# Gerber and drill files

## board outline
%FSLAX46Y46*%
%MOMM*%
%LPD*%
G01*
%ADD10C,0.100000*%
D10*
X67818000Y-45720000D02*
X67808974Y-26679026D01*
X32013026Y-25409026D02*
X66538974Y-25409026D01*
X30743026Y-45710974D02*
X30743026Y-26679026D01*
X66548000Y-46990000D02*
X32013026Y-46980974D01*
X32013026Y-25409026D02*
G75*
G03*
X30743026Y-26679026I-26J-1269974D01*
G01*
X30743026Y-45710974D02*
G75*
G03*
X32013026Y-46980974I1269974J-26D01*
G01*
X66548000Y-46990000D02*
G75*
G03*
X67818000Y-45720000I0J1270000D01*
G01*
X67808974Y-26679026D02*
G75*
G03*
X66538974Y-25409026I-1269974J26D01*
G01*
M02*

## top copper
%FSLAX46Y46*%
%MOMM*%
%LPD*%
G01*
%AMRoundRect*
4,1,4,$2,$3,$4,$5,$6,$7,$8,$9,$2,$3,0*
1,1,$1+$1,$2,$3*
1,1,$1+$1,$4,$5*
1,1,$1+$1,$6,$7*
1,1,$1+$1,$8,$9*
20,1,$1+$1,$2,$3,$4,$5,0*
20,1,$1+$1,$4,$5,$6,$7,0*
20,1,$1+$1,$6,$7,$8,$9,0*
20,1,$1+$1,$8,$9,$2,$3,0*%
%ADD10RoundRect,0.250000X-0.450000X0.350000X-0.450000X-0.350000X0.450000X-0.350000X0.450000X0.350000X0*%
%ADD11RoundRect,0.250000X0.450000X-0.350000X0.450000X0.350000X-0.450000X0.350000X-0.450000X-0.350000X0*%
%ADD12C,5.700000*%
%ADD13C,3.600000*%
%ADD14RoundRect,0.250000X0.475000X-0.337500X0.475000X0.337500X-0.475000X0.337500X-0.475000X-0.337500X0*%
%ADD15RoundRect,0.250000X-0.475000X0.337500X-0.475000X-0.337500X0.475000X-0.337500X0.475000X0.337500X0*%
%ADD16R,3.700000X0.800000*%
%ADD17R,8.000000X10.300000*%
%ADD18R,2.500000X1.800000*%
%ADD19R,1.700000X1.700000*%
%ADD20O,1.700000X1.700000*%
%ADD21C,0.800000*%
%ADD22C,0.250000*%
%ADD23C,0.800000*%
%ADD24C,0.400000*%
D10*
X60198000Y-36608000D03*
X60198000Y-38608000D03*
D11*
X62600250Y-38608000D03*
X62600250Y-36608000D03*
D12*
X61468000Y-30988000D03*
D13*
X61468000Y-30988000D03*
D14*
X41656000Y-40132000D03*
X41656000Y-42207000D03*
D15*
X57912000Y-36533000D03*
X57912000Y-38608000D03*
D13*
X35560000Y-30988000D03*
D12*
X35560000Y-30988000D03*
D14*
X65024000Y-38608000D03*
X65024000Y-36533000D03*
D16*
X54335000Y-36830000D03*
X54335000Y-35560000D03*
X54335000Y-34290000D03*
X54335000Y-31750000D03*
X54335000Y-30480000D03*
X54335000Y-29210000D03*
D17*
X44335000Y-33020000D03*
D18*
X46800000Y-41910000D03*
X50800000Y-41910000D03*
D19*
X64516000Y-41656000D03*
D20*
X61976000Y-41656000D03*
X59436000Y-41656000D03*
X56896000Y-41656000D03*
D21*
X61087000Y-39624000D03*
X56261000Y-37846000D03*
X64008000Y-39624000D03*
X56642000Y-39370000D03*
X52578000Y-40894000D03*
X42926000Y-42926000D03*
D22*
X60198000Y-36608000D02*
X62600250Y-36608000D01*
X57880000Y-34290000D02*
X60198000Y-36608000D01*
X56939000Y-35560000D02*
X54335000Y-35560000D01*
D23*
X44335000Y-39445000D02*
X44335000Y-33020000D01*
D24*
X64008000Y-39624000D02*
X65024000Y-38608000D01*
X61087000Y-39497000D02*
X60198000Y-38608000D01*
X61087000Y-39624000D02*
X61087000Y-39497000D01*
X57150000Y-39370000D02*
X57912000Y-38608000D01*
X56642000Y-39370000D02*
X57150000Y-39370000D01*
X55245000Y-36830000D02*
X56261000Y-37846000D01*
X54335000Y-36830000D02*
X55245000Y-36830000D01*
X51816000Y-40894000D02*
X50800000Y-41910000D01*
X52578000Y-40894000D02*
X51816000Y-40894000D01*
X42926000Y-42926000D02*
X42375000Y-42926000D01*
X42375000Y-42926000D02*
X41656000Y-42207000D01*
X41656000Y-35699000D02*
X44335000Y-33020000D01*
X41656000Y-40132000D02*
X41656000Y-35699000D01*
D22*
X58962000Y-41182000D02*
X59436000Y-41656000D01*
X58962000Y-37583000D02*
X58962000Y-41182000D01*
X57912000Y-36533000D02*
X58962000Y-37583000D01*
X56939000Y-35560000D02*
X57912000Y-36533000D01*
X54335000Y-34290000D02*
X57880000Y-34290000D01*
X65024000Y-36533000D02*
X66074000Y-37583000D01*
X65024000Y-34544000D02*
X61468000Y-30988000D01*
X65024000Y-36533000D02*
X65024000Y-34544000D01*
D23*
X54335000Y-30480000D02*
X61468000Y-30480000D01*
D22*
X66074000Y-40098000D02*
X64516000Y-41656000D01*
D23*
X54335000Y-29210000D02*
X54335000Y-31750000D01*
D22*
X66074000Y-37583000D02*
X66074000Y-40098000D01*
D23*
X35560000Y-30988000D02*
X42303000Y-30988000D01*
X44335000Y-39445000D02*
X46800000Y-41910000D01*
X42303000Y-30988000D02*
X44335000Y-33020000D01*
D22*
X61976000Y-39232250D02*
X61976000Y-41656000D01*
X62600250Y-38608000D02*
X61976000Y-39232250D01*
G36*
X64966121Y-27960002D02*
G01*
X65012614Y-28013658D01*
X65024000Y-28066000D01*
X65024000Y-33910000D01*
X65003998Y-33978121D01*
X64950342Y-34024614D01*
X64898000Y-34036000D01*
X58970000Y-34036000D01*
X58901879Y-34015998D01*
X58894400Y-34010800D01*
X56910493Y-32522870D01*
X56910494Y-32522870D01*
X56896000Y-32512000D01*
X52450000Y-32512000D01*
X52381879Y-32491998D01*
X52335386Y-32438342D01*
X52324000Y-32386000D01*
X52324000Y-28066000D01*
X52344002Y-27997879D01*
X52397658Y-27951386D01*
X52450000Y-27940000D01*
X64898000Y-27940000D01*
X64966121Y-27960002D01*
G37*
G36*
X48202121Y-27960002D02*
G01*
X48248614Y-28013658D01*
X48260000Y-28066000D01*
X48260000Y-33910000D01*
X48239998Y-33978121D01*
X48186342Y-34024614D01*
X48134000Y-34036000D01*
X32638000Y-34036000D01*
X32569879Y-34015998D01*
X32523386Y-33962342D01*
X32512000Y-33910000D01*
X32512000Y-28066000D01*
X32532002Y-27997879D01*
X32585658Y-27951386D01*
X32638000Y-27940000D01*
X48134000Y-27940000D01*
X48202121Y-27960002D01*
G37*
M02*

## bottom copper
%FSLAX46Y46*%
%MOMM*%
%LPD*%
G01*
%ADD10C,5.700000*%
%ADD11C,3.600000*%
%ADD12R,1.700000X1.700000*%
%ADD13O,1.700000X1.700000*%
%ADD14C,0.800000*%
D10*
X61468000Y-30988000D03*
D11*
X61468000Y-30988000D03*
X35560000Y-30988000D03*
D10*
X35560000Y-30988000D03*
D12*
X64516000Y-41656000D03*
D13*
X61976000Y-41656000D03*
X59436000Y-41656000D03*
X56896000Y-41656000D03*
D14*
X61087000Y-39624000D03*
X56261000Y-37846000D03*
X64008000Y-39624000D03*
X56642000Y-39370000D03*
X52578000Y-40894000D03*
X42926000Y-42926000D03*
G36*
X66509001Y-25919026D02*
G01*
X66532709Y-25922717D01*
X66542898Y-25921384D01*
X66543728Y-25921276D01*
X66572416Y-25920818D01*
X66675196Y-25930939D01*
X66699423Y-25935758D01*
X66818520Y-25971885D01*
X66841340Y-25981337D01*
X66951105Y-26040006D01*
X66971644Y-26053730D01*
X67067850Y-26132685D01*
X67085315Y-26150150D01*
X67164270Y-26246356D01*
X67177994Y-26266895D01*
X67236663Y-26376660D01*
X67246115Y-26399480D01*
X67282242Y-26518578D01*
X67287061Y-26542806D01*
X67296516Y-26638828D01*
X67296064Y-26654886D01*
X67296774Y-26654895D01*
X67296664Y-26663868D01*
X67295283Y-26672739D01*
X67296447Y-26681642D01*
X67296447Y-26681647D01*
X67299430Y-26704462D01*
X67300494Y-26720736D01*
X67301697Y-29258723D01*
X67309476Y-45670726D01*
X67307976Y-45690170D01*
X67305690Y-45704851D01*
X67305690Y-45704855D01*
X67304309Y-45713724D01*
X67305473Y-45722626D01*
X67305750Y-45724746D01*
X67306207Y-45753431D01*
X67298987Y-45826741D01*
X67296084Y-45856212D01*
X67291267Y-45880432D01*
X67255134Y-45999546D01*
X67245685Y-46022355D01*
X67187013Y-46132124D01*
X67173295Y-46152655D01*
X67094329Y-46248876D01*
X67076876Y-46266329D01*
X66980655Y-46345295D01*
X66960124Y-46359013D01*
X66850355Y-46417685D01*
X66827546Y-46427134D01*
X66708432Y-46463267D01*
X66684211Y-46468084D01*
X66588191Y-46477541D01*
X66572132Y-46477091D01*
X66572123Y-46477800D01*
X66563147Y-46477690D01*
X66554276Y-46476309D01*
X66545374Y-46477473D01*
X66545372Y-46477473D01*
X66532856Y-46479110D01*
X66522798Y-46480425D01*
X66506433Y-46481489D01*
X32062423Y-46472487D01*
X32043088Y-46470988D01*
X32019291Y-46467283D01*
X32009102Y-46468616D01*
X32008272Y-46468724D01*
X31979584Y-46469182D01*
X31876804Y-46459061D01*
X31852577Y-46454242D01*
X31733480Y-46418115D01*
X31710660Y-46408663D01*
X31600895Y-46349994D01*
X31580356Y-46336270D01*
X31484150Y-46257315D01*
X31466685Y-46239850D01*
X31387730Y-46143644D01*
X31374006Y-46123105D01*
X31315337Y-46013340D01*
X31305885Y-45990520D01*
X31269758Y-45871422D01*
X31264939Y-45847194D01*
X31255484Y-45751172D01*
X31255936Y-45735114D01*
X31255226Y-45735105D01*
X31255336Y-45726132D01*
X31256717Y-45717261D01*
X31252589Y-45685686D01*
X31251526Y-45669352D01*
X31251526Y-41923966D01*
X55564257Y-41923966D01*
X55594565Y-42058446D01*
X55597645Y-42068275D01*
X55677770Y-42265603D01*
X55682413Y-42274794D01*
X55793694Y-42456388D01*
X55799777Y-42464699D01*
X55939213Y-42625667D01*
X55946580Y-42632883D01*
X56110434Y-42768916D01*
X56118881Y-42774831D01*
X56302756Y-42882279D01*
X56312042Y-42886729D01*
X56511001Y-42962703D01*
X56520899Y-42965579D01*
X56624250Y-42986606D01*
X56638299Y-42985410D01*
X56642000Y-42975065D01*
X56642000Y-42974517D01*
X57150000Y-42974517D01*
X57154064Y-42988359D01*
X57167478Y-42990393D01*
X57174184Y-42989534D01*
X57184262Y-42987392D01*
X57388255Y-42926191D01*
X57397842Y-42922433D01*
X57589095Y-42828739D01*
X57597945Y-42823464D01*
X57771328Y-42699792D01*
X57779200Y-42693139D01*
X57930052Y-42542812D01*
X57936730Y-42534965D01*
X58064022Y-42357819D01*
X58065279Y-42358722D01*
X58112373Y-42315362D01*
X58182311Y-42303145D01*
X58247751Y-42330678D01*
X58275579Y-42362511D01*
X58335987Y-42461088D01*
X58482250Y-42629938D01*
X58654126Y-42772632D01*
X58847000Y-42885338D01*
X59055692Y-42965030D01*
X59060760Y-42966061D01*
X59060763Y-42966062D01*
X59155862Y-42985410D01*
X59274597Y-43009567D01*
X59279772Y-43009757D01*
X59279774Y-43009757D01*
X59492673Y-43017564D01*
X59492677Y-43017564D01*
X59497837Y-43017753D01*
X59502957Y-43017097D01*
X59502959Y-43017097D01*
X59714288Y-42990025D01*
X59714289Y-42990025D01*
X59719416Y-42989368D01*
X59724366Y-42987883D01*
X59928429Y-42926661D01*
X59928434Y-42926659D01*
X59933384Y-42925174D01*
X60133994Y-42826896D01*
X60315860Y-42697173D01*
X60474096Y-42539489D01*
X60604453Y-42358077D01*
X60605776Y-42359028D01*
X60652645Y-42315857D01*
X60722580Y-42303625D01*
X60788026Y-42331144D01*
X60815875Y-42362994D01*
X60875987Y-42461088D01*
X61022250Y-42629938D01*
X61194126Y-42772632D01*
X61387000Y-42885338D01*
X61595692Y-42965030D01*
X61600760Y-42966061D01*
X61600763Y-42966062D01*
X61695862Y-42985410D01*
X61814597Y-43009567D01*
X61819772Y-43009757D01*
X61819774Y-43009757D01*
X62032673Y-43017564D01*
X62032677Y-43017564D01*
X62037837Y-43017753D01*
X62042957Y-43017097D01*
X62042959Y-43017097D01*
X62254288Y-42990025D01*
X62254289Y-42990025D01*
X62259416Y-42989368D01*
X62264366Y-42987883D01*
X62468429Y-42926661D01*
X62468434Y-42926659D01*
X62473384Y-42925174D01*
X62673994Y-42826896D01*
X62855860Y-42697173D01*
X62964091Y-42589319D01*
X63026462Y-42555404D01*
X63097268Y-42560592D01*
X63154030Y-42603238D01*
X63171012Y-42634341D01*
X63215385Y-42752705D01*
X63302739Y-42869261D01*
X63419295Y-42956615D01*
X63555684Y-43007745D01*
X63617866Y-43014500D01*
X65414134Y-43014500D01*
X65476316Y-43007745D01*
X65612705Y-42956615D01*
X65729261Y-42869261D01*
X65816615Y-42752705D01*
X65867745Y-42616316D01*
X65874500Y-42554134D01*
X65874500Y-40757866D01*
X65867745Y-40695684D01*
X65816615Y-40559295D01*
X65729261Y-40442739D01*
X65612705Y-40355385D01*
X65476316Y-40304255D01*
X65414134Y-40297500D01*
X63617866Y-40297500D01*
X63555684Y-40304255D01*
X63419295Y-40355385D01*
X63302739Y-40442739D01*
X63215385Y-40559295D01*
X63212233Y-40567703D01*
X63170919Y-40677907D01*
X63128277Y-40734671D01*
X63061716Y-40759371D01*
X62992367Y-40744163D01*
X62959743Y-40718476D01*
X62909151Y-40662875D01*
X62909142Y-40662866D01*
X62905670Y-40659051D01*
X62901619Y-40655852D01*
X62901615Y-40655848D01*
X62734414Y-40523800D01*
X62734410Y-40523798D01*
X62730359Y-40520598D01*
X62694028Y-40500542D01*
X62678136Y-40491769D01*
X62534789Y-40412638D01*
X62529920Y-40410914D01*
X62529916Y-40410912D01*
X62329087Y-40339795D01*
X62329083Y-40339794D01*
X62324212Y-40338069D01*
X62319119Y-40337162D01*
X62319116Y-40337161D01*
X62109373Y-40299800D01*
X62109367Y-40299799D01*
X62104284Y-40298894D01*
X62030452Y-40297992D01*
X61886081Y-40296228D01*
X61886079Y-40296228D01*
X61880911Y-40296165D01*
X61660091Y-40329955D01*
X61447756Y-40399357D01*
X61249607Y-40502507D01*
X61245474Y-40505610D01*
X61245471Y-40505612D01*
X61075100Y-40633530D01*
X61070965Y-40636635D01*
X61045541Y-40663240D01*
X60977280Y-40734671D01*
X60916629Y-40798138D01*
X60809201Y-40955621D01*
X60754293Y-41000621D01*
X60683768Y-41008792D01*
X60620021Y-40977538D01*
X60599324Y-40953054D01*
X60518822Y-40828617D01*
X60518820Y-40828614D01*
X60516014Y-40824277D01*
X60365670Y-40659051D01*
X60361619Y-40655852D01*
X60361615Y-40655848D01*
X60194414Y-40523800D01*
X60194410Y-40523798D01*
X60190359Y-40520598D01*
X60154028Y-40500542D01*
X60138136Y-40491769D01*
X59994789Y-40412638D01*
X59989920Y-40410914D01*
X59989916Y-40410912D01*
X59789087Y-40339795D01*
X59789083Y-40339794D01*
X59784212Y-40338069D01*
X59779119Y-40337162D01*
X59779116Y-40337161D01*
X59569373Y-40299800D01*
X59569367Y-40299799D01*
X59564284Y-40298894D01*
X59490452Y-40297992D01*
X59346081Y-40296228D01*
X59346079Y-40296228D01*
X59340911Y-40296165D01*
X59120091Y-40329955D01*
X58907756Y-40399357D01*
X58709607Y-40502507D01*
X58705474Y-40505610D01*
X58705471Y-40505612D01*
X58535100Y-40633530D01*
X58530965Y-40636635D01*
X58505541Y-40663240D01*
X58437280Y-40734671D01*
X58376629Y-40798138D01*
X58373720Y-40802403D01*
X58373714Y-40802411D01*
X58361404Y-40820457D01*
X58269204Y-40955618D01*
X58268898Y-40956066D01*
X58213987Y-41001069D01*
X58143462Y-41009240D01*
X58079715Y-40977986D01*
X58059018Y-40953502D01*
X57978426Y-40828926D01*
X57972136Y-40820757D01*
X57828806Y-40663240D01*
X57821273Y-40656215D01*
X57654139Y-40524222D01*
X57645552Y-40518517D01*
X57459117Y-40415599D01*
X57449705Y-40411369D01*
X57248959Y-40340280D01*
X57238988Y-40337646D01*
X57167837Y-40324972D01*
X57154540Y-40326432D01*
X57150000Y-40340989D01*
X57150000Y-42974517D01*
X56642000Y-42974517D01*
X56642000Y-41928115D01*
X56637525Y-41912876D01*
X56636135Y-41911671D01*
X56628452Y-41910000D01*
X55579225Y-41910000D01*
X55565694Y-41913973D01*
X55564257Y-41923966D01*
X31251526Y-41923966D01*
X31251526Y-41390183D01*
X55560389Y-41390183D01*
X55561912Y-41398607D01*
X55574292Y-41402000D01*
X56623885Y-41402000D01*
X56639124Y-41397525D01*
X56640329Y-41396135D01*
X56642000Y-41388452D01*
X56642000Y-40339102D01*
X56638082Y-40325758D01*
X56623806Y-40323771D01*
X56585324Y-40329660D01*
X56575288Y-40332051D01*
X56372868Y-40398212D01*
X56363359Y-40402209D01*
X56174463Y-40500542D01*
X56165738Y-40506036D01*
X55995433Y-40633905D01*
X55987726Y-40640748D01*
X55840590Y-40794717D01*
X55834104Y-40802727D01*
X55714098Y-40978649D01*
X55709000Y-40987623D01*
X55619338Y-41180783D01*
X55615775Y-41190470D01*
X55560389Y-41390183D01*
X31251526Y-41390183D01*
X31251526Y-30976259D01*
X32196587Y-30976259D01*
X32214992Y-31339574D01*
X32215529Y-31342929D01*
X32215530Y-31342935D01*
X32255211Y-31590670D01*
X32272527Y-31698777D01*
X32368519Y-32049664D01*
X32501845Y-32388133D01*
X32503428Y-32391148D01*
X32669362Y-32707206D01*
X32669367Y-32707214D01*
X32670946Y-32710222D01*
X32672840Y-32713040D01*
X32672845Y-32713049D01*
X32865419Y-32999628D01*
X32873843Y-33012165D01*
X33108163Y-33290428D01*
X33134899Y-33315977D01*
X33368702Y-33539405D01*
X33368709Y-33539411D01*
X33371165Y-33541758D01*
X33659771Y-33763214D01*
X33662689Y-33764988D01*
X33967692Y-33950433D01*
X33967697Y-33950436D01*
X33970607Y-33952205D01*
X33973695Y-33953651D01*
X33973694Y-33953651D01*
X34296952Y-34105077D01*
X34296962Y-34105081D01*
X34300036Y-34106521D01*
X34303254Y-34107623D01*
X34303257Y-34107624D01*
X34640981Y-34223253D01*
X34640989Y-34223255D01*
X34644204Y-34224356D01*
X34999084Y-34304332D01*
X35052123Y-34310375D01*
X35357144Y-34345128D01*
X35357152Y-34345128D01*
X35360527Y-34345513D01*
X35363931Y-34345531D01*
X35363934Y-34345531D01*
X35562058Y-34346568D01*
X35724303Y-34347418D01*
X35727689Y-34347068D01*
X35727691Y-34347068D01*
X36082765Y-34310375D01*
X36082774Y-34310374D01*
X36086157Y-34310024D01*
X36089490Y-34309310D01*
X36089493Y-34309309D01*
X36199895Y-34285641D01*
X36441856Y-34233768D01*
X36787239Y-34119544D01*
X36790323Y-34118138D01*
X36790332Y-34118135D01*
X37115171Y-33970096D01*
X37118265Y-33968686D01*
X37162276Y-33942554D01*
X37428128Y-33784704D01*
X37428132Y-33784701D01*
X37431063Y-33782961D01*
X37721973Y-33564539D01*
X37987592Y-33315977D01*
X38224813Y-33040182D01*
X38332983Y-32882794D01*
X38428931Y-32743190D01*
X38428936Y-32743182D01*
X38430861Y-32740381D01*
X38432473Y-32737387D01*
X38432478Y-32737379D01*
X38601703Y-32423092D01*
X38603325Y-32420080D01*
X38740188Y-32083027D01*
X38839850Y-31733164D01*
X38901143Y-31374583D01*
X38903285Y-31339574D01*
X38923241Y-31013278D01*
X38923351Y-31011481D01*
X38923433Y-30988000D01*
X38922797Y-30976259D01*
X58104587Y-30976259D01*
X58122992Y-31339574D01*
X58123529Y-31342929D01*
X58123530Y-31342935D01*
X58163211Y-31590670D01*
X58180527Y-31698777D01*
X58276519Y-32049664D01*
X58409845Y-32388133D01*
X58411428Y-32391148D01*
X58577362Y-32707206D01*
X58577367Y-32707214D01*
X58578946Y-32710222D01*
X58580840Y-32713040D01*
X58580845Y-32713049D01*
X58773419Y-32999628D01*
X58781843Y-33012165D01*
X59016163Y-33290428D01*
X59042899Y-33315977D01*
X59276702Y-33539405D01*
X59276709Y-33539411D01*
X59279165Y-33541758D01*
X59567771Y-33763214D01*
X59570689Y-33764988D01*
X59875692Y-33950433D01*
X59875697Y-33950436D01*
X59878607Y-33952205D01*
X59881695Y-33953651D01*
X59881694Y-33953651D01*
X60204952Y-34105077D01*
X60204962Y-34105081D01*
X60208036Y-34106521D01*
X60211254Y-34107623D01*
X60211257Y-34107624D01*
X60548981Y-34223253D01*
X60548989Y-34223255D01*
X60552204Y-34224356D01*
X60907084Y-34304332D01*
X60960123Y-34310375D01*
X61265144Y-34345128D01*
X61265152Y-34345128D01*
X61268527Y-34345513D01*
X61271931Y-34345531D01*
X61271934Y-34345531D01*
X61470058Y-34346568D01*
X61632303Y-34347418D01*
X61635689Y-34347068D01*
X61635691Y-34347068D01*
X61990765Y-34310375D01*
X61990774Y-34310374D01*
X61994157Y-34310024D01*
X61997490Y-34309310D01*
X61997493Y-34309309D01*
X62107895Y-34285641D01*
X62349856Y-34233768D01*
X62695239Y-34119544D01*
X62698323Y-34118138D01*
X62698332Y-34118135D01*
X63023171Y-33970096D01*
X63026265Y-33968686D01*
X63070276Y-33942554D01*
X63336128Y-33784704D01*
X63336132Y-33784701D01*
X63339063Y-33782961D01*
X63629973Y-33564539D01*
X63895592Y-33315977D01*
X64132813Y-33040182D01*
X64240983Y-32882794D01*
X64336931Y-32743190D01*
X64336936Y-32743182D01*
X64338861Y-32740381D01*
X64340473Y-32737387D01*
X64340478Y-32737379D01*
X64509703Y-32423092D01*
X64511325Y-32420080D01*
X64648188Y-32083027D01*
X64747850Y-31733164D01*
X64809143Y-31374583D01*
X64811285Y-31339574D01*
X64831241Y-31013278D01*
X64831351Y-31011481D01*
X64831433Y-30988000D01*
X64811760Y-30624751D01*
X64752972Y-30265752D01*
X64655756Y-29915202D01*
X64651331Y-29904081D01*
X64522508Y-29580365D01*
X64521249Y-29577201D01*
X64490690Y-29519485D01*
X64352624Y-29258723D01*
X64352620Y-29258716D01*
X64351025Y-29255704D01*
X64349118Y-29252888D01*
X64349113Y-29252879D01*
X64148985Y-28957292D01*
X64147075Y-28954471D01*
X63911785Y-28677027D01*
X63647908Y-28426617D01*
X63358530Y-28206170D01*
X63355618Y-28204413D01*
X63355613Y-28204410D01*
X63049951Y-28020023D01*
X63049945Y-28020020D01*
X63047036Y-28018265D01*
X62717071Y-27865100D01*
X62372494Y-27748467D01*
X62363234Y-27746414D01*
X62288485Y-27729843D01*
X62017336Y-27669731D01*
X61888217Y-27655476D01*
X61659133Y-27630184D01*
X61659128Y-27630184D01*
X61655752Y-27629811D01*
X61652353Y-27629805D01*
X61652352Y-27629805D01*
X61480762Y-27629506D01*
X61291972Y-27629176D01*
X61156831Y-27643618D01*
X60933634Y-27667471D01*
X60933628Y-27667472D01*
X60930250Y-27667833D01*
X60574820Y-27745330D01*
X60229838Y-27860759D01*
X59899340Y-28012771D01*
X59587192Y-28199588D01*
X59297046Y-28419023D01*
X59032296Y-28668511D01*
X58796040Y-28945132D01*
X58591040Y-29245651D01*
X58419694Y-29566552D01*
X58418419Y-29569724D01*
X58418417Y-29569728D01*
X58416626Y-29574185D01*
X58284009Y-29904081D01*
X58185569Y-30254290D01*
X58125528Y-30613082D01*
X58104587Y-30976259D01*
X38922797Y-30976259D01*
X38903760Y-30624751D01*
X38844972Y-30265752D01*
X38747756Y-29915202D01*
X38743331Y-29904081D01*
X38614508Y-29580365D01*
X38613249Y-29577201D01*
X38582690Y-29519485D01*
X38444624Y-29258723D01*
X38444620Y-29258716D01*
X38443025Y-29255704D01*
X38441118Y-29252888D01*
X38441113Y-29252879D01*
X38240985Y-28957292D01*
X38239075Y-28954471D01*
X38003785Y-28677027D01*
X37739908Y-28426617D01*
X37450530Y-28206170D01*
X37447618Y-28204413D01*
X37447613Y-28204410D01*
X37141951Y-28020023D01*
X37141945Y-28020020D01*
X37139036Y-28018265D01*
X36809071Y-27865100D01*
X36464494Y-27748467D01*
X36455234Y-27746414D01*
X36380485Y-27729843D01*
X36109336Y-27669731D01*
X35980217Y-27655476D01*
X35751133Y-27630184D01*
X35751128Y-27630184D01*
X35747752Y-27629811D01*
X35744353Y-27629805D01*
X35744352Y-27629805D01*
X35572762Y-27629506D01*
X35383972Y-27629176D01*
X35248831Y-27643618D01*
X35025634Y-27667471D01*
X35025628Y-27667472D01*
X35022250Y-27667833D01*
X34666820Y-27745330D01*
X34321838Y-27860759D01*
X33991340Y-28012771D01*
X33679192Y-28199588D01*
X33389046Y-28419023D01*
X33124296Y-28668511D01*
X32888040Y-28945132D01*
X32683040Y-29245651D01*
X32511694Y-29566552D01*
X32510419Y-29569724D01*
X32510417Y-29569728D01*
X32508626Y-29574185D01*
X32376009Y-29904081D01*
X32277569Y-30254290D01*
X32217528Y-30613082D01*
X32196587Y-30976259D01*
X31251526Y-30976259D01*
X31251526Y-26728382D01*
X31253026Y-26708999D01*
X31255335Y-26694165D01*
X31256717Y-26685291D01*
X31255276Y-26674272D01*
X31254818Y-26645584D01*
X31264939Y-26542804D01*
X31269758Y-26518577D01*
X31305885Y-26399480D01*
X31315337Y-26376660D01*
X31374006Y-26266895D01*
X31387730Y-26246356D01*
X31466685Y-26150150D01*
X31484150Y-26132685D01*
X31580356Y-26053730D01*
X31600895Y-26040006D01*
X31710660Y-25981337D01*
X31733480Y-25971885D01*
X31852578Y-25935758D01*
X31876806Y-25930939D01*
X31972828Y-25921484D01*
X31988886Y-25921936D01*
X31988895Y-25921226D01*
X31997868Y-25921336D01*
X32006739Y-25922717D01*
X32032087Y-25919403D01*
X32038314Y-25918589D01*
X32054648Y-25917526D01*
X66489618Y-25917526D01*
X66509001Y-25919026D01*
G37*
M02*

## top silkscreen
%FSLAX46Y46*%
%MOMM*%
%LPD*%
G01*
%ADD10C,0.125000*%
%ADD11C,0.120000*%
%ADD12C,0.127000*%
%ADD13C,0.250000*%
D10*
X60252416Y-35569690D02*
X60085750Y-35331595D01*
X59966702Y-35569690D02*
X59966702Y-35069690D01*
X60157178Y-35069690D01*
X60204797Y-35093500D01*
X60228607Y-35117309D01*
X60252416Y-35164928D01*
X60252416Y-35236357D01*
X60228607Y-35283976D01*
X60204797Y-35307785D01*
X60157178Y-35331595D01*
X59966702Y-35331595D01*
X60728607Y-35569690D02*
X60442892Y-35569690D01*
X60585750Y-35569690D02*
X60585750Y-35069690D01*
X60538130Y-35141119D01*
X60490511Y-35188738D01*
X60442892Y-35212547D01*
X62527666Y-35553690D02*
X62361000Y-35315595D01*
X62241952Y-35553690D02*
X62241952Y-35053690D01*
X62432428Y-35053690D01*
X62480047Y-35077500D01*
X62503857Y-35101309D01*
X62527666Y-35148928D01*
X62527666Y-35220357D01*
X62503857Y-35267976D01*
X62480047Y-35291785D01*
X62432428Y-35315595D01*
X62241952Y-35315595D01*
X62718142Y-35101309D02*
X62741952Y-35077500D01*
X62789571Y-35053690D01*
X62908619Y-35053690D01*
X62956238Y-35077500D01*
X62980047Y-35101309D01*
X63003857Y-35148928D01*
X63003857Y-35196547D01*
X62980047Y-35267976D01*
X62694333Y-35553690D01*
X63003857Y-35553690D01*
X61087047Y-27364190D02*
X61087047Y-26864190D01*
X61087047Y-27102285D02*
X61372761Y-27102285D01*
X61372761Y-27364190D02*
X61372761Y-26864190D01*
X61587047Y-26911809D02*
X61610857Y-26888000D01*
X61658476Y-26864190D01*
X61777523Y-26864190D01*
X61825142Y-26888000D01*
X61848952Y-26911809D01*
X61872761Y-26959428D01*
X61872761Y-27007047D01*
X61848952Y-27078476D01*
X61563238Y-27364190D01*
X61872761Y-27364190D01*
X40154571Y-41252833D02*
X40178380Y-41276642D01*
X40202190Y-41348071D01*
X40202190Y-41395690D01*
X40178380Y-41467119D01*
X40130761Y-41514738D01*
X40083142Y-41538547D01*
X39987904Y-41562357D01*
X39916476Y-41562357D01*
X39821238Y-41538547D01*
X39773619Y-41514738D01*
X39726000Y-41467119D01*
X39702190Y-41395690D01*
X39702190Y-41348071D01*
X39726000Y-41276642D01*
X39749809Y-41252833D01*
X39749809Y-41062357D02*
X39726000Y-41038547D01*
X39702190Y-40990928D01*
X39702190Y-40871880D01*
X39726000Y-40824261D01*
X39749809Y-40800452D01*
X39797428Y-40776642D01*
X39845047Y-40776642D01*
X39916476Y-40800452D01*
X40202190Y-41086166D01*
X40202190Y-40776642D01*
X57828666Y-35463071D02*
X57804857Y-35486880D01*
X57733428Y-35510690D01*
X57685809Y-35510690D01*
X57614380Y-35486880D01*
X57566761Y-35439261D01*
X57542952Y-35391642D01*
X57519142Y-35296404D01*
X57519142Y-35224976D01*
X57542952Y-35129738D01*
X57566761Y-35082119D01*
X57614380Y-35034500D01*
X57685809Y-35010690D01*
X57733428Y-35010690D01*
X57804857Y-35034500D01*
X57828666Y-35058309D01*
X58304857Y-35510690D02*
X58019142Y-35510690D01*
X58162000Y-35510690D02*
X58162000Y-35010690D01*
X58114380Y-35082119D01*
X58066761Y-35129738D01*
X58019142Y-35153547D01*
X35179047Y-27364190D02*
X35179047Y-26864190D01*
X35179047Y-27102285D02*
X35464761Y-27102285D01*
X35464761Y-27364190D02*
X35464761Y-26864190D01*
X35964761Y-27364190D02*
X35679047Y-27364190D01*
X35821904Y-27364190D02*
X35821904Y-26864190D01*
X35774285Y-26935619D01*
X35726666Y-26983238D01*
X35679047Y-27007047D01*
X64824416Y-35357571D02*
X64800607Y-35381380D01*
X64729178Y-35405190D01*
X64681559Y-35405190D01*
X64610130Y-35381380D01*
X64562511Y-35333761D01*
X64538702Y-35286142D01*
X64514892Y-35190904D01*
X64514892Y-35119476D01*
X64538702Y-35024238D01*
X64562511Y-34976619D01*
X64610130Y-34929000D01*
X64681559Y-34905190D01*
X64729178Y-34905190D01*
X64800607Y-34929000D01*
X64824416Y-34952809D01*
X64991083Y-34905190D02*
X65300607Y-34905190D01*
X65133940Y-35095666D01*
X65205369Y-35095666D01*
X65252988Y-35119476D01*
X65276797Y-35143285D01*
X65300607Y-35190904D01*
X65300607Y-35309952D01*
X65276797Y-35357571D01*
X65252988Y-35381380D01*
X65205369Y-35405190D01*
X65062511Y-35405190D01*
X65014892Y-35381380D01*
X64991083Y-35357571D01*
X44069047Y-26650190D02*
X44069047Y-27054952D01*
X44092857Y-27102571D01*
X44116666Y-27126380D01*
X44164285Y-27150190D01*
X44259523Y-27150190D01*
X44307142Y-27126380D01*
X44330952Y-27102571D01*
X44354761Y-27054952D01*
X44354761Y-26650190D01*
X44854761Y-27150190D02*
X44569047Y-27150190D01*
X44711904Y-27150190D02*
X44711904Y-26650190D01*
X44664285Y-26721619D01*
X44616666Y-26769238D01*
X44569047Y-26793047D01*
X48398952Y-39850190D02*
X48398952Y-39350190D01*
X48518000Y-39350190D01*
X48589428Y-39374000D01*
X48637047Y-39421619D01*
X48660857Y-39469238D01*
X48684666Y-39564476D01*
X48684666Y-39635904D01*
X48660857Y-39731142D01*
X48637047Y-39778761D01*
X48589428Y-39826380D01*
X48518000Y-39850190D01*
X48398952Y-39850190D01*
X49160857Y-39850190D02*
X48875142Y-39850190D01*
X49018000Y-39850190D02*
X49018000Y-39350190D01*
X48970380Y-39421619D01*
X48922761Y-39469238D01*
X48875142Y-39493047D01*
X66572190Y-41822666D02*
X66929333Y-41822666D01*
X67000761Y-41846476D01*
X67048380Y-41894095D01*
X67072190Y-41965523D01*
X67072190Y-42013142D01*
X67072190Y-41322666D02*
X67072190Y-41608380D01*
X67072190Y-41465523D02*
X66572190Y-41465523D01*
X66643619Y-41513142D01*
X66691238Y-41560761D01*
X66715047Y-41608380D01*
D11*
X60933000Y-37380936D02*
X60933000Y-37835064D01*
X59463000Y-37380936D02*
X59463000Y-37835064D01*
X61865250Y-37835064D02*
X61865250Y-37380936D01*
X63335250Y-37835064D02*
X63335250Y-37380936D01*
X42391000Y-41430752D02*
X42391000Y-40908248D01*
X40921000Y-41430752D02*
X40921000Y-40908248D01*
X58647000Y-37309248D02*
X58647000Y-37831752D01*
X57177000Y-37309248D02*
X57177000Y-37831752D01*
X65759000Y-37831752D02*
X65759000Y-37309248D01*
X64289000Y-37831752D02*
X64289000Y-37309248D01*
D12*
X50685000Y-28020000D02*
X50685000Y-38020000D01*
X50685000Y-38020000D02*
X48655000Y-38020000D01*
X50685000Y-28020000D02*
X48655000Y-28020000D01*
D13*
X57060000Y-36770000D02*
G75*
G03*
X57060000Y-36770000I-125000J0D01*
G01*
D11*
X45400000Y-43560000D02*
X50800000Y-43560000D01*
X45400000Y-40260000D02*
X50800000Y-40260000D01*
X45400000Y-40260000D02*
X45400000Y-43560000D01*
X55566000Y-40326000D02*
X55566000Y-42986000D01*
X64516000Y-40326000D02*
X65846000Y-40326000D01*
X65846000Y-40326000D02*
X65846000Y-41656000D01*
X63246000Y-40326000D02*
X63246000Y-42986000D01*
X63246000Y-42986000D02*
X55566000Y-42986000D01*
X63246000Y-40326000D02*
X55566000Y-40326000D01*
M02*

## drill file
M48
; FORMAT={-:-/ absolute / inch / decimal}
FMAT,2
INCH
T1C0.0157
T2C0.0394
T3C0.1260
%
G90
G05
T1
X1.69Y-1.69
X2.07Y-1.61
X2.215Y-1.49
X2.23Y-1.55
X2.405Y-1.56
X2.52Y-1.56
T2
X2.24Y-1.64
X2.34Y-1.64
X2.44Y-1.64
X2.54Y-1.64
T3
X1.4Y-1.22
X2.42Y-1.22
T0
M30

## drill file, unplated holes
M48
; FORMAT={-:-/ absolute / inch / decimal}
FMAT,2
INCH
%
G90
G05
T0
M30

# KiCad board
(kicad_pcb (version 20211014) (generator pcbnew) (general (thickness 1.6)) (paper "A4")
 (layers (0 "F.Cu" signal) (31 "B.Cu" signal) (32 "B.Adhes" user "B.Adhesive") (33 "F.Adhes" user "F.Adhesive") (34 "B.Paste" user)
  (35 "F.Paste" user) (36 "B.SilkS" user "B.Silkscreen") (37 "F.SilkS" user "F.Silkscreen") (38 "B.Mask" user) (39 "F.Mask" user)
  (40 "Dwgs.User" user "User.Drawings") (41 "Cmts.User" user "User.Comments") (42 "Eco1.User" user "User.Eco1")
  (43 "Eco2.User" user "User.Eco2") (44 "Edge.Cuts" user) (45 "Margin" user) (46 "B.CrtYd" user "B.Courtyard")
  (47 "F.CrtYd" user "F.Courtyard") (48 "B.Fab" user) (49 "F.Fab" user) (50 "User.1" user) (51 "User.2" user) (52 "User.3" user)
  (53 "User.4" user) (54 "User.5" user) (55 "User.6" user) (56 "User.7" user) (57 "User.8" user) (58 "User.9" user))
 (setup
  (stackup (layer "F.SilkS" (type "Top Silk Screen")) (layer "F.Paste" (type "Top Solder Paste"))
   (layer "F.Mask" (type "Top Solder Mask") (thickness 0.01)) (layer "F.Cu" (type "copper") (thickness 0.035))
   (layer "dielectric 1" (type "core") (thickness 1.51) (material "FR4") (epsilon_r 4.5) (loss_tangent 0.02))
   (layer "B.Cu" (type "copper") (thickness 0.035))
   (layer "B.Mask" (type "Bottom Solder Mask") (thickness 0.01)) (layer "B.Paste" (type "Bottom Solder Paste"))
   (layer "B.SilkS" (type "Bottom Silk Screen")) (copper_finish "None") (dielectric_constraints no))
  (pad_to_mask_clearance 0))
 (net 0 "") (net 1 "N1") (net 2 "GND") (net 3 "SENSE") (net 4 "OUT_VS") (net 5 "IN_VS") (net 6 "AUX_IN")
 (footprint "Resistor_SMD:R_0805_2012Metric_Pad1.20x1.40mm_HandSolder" (layer "F.Cu") (at 60.198 37.608 -90)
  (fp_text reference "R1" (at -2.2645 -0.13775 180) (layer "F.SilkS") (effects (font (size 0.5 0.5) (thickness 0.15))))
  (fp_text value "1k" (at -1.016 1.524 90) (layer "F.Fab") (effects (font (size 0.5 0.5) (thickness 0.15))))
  (fp_line (start -0.227064 -0.735) (end 0.227064 -0.735) (layer "F.SilkS") (width 0.12))
  (fp_line (start -0.227064 0.735) (end 0.227064 0.735) (layer "F.SilkS") (width 0.12))
  (pad "1" smd roundrect (at -1 0 270) (size 1.2 1.4) (layers "F.Cu" "F.Paste" "F.Mask") (roundrect_rratio 0.2083333333) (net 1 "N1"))
  (pad "2" smd roundrect (at 1 0 270) (size 1.2 1.4) (layers "F.Cu" "F.Paste" "F.Mask") (roundrect_rratio 0.2083333333) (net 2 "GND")))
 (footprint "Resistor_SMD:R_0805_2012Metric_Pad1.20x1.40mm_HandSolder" (layer "F.Cu") (at 62.60025 37.608 90)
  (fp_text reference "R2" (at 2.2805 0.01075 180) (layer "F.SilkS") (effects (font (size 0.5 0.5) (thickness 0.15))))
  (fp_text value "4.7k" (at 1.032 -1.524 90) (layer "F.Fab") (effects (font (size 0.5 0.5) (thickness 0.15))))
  (fp_line (start -0.227064 -0.735) (end 0.227064 -0.735) (layer "F.SilkS") (width 0.12))
  (fp_line (start -0.227064 0.735) (end 0.227064 0.735) (layer "F.SilkS") (width 0.12))
  (pad "1" smd roundrect (at -1 0 90) (size 1.2 1.4) (layers "F.Cu" "F.Paste" "F.Mask") (roundrect_rratio 0.2083333333) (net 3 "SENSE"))
  (pad "2" smd roundrect (at 1 0 90) (size 1.2 1.4) (layers "F.Cu" "F.Paste" "F.Mask") (roundrect_rratio 0.2083333333) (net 1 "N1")))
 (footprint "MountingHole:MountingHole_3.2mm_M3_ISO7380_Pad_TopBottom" (layer "F.Cu") (at 61.468 30.988)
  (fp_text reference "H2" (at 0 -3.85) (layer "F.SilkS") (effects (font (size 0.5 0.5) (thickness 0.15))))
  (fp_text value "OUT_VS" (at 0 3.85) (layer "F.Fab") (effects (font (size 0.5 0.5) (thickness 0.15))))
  (pad "1" connect circle (at 0 0) (size 5.7 5.7) (layers "B.Cu" "B.Mask") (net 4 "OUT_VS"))
  (pad "1" connect circle (at 0 0) (size 5.7 5.7) (layers "F.Cu" "F.Mask") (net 4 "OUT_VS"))
  (pad "1" thru_hole circle (at 0 0) (size 3.6 3.6) (drill 3.2) (layers *.Cu *.Mask) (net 4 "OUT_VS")))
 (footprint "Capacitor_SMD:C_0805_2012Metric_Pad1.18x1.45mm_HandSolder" (layer "F.Cu") (at 41.656 41.1695 90)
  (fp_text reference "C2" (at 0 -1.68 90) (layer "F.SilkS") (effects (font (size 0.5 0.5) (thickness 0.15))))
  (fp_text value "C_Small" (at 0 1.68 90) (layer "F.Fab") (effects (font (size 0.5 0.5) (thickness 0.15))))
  (fp_line (start -0.261252 -0.735) (end 0.261252 -0.735) (layer "F.SilkS") (width 0.12))
  (fp_line (start -0.261252 0.735) (end 0.261252 0.735) (layer "F.SilkS") (width 0.12))
  (pad "1" smd roundrect (at -1.0375 0 90) (size 1.175 1.45) (layers "F.Cu" "F.Paste" "F.Mask") (roundrect_rratio 0.2127659574)
   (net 2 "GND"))
  (pad "2" smd roundrect (at 1.0375 0 90) (size 1.175 1.45) (layers "F.Cu" "F.Paste" "F.Mask") (roundrect_rratio 0.2127659574)
   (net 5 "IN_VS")))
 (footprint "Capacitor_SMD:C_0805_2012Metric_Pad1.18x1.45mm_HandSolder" (layer "F.Cu") (at 57.912 37.5705 -90)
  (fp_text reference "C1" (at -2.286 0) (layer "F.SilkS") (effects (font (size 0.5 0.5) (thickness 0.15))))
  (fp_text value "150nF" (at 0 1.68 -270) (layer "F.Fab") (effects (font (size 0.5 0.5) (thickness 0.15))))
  (fp_line (start -0.261252 -0.735) (end 0.261252 -0.735) (layer "F.SilkS") (width 0.12))
  (fp_line (start -0.261252 0.735) (end 0.261252 0.735) (layer "F.SilkS") (width 0.12))
  (pad "1" smd roundrect (at -1.0375 0 270) (size 1.175 1.45) (layers "F.Cu" "F.Paste" "F.Mask") (roundrect_rratio 0.2127659574)
   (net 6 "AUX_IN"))
  (pad "2" smd roundrect (at 1.0375 0 270) (size 1.175 1.45) (layers "F.Cu" "F.Paste" "F.Mask") (roundrect_rratio 0.2127659574)
   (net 2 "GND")))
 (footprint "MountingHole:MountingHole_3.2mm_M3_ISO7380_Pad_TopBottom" (layer "F.Cu") (at 35.56 30.988)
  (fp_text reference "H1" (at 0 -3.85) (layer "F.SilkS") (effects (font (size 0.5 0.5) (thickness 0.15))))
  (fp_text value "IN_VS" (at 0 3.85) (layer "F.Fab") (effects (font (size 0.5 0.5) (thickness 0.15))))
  (pad "1" thru_hole circle (at 0 0) (size 3.6 3.6) (drill 3.2) (layers *.Cu *.Mask) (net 5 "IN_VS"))
  (pad "1" connect circle (at 0 0) (size 5.7 5.7) (layers "B.Cu" "B.Mask") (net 5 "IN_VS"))
  (pad "1" connect circle (at 0 0) (size 5.7 5.7) (layers "F.Cu" "F.Mask") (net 5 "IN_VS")))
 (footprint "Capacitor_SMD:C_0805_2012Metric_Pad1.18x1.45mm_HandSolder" (layer "F.Cu") (at 65.024 37.5705 90)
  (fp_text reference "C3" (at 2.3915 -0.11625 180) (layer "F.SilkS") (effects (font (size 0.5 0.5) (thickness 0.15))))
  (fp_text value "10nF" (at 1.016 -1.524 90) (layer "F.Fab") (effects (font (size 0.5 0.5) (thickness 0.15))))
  (fp_line (start -0.261252 0.735) (end 0.261252 0.735) (layer "F.SilkS") (width 0.12))
  (fp_line (start -0.261252 -0.735) (end 0.261252 -0.735) (layer "F.SilkS") (width 0.12))
  (pad "1" smd roundrect (at -1.0375 0 90) (size 1.175 1.45) (layers "F.Cu" "F.Paste" "F.Mask") (roundrect_rratio 0.2127659574)
   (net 2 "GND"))
  (pad "2" smd roundrect (at 1.0375 0 90) (size 1.175 1.45) (layers "F.Cu" "F.Paste" "F.Mask") (roundrect_rratio 0.2127659574)
   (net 4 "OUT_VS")))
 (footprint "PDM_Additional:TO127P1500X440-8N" (layer "F.Cu") (at 48.26 33.02 180)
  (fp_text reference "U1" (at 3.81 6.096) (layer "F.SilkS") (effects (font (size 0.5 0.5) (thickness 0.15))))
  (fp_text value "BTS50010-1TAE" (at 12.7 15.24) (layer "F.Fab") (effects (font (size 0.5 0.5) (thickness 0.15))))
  (fp_line (start -2.425 5) (end -2.425 -5) (layer "F.SilkS") (width 0.127))
  (fp_line (start -2.425 -5) (end -0.395 -5) (layer "F.SilkS") (width 0.127))
  (fp_line (start -2.425 5) (end -0.395 5) (layer "F.SilkS") (width 0.127))
  (fp_circle (center -8.675 -3.75) (end -8.55 -3.75) (layer "F.SilkS") (width 0.25) (fill none))
  (pad "1" smd rect (at -6.075 -3.81 180) (size 3.7 0.8) (layers "F.Cu" "F.Paste" "F.Mask") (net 2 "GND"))
  (pad "2" smd rect (at -6.075 -2.54 180) (size 3.7 0.8) (layers "F.Cu" "F.Paste" "F.Mask") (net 6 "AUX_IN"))
  (pad "3" smd rect (at -6.075 -1.27 180) (size 3.7 0.8) (layers "F.Cu" "F.Paste" "F.Mask") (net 1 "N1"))
  (pad "5" smd rect (at -6.075 1.27 180) (size 3.7 0.8) (layers "F.Cu" "F.Paste" "F.Mask") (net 4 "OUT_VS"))
  (pad "6" smd rect (at -6.075 2.54 180) (size 3.7 0.8) (layers "F.Cu" "F.Paste" "F.Mask") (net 4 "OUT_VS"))
  (pad "7" smd rect (at -6.075 3.81 180) (size 3.7 0.8) (layers "F.Cu" "F.Paste" "F.Mask") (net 4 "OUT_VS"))
  (pad "8" smd rect (at 3.925 0 270) (size 10.3 8) (layers "F.Cu" "F.Mask") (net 5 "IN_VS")))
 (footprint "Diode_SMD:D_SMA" (layer "F.Cu") (at 48.8 41.91)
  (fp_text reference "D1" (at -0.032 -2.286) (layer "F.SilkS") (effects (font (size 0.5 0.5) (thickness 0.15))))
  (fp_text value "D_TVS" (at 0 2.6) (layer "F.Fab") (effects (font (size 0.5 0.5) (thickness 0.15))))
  (fp_line (start -3.4 1.65) (end 2 1.65) (layer "F.SilkS") (width 0.12))
  (fp_line (start -3.4 -1.65) (end 2 -1.65) (layer "F.SilkS") (width 0.12))
  (fp_line (start -3.4 -1.65) (end -3.4 1.65) (layer "F.SilkS") (width 0.12))
  (pad "1" smd rect (at -2 0) (size 2.5 1.8) (layers "F.Cu" "F.Paste" "F.Mask") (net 5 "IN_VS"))
  (pad "2" smd rect (at 2 0) (size 2.5 1.8) (layers "F.Cu" "F.Paste" "F.Mask") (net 2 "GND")))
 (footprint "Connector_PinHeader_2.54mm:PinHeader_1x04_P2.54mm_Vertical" (layer "F.Cu") (at 64.516 41.656 -90)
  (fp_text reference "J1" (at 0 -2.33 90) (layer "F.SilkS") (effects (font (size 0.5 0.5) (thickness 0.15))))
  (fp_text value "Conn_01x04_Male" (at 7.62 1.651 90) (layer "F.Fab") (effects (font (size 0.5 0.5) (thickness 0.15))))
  (fp_line (start -1.33 8.95) (end 1.33 8.95) (layer "F.SilkS") (width 0.12))
  (fp_line (start -1.33 0) (end -1.33 -1.33) (layer "F.SilkS") (width 0.12))
  (fp_line (start -1.33 -1.33) (end 0 -1.33) (layer "F.SilkS") (width 0.12))
  (fp_line (start -1.33 1.27) (end 1.33 1.27) (layer "F.SilkS") (width 0.12))
  (fp_line (start 1.33 1.27) (end 1.33 8.95) (layer "F.SilkS") (width 0.12))
  (fp_line (start -1.33 1.27) (end -1.33 8.95) (layer "F.SilkS") (width 0.12))
  (pad "1" thru_hole rect (at 0 0 270) (size 1.7 1.7) (drill 1) (layers *.Cu *.Mask) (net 4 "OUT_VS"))
  (pad "2" thru_hole oval (at 0 2.54 270) (size 1.7 1.7) (drill 1) (layers *.Cu *.Mask) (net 3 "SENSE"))
  (pad "3" thru_hole oval (at 0 5.08 270) (size 1.7 1.7) (drill 1) (layers *.Cu *.Mask) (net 6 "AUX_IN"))
  (pad "4" thru_hole oval (at 0 7.62 270) (size 1.7 1.7) (drill 1) (layers *.Cu *.Mask) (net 2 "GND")))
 (gr_line (start 32.013026 25.409026) (end 66.538974 25.409026) (layer "Edge.Cuts") (width 0.1))
 (gr_arc (start 30.743026 26.679026) (mid 31.115 25.781) (end 32.013026 25.409026) (layer "Edge.Cuts") (width 0.1))
 (gr_line (start 30.743026 45.710974) (end 30.743026 26.679026) (layer "Edge.Cuts") (width 0.1))
 (gr_arc (start 32.013026 46.980974) (mid 31.115 46.609) (end 30.743026 45.710974) (layer "Edge.Cuts") (width 0.1))
 (gr_line (start 67.818 45.72) (end 67.808974 26.679026) (layer "Edge.Cuts") (width 0.1))
 (gr_line (start 66.548 46.99) (end 32.013026 46.980974) (layer "Edge.Cuts") (width 0.1))
 (gr_arc (start 67.818 45.72) (mid 67.446026 46.618026) (end 66.548 46.99) (layer "Edge.Cuts") (width 0.1))
 (gr_arc (start 66.538974 25.409026) (mid 67.437 25.781) (end 67.808974 26.679026) (layer "Edge.Cuts") (width 0.1))
 (segment (start 54.335 36.83) (end 55.245 36.83) (width 0.4) (layer "F.Cu") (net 2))
 (segment (start 57.15 39.37) (end 57.912 38.608) (width 0.4) (layer "F.Cu") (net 2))
 (segment (start 64.008 39.624) (end 65.024 38.608) (width 0.4) (layer "F.Cu") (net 2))
 (segment (start 42.926 42.926) (end 42.375 42.926) (width 0.4) (layer "F.Cu") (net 2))
 (segment (start 61.087 39.624) (end 61.087 39.497) (width 0.4) (layer "F.Cu") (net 2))
 (segment (start 42.375 42.926) (end 41.656 42.207) (width 0.4) (layer "F.Cu") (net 2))
 (segment (start 51.816 40.894) (end 50.8 41.91) (width 0.4) (layer "F.Cu") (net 2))
 (segment (start 56.642 39.37) (end 57.15 39.37) (width 0.4) (layer "F.Cu") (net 2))
 (segment (start 55.245 36.83) (end 56.261 37.846) (width 0.4) (layer "F.Cu") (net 2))
 (segment (start 52.578 40.894) (end 51.816 40.894) (width 0.4) (layer "F.Cu") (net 2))
 (segment (start 61.087 39.497) (end 60.198 38.608) (width 0.4) (layer "F.Cu") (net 2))
 (via (at 42.926 42.926) (size 0.8) (drill 0.4) (layers "F.Cu" "B.Cu") (free) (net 2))
 (via (at 52.578 40.894) (size 0.8) (drill 0.4) (layers "F.Cu" "B.Cu") (free) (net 2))
 (via (at 64.008 39.624) (size 0.8) (drill 0.4) (layers "F.Cu" "B.Cu") (free) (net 2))
 (via (at 56.642 39.37) (size 0.8) (drill 0.4) (layers "F.Cu" "B.Cu") (free) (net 2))
 (via (at 56.261 37.846) (size 0.8) (drill 0.4) (layers "F.Cu" "B.Cu") (free) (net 2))
 (via (at 61.087 39.624) (size 0.8) (drill 0.4) (layers "F.Cu" "B.Cu") (free) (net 2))
 (segment (start 58.962 41.182) (end 59.436 41.656) (width 0.25) (layer "F.Cu") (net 6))
 (segment (start 58.962 37.583) (end 58.962 41.182) (width 0.25) (layer "F.Cu") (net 6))
 (segment (start 57.912 36.533) (end 58.962 37.583) (width 0.25) (layer "F.Cu") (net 6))
 (segment (start 56.939 35.56) (end 54.335 35.56) (width 0.25) (layer "F.Cu") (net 6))
 (segment (start 56.939 35.56) (end 57.912 36.533) (width 0.25) (layer "F.Cu") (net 6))
 (segment (start 60.198 36.608) (end 62.60025 36.608) (width 0.25) (layer "F.Cu") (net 1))
 (segment (start 54.335 34.29) (end 57.88 34.29) (width 0.25) (layer "F.Cu") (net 1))
 (segment (start 57.88 34.29) (end 60.198 36.608) (width 0.25) (layer "F.Cu") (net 1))
 (segment (start 65.024 36.533) (end 66.074 37.583) (width 0.25) (layer "F.Cu") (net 4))
 (segment (start 65.024 34.544) (end 61.468 30.988) (width 0.25) (layer "F.Cu") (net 4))
 (segment (start 65.024 36.533) (end 65.024 34.544) (width 0.25) (layer "F.Cu") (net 4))
 (segment (start 54.335 30.48) (end 61.468 30.48) (width 0.8) (layer "F.Cu") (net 4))
 (segment (start 66.074 40.098) (end 64.516 41.656) (width 0.25) (layer "F.Cu") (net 4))
 (segment (start 54.335 29.21) (end 54.335 31.75) (width 0.8) (layer "F.Cu") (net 4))
 (segment (start 66.074 37.583) (end 66.074 40.098) (width 0.25) (layer "F.Cu") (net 4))
 (segment (start 35.56 30.988) (end 42.303 30.988) (width 0.8) (layer "F.Cu") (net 5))
 (segment (start 44.335 39.445) (end 44.335 33.02) (width 0.8) (layer "F.Cu") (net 5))
 (segment (start 41.656 35.699) (end 44.335 33.02) (width 0.4) (layer "F.Cu") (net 5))
 (segment (start 44.335 39.445) (end 46.8 41.91) (width 0.8) (layer "F.Cu") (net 5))
 (segment (start 41.656 40.132) (end 41.656 35.699) (width 0.4) (layer "F.Cu") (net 5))
 (segment (start 42.303 30.988) (end 44.335 33.02) (width 0.8) (layer "F.Cu") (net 5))
 (segment (start 61.976 39.23225) (end 61.976 41.656) (width 0.25) (layer "F.Cu") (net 3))
 (segment (start 62.60025 38.608) (end 61.976 39.23225) (width 0.25) (layer "F.Cu") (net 3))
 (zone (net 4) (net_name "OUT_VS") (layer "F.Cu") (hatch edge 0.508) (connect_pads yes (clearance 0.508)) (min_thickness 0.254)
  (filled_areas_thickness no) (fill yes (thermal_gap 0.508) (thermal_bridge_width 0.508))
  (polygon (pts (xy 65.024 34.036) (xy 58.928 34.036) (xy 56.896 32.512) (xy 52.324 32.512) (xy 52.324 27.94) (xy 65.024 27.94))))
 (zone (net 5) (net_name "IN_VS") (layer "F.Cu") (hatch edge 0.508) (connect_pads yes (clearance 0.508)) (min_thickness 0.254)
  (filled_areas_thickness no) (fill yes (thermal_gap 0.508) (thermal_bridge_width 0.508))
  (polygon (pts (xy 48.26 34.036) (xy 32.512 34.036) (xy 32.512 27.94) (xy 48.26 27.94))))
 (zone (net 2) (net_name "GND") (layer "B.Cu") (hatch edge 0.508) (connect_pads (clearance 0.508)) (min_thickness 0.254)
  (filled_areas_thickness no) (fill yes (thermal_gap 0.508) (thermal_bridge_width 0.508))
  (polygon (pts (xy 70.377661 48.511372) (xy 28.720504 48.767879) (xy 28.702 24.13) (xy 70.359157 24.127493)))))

